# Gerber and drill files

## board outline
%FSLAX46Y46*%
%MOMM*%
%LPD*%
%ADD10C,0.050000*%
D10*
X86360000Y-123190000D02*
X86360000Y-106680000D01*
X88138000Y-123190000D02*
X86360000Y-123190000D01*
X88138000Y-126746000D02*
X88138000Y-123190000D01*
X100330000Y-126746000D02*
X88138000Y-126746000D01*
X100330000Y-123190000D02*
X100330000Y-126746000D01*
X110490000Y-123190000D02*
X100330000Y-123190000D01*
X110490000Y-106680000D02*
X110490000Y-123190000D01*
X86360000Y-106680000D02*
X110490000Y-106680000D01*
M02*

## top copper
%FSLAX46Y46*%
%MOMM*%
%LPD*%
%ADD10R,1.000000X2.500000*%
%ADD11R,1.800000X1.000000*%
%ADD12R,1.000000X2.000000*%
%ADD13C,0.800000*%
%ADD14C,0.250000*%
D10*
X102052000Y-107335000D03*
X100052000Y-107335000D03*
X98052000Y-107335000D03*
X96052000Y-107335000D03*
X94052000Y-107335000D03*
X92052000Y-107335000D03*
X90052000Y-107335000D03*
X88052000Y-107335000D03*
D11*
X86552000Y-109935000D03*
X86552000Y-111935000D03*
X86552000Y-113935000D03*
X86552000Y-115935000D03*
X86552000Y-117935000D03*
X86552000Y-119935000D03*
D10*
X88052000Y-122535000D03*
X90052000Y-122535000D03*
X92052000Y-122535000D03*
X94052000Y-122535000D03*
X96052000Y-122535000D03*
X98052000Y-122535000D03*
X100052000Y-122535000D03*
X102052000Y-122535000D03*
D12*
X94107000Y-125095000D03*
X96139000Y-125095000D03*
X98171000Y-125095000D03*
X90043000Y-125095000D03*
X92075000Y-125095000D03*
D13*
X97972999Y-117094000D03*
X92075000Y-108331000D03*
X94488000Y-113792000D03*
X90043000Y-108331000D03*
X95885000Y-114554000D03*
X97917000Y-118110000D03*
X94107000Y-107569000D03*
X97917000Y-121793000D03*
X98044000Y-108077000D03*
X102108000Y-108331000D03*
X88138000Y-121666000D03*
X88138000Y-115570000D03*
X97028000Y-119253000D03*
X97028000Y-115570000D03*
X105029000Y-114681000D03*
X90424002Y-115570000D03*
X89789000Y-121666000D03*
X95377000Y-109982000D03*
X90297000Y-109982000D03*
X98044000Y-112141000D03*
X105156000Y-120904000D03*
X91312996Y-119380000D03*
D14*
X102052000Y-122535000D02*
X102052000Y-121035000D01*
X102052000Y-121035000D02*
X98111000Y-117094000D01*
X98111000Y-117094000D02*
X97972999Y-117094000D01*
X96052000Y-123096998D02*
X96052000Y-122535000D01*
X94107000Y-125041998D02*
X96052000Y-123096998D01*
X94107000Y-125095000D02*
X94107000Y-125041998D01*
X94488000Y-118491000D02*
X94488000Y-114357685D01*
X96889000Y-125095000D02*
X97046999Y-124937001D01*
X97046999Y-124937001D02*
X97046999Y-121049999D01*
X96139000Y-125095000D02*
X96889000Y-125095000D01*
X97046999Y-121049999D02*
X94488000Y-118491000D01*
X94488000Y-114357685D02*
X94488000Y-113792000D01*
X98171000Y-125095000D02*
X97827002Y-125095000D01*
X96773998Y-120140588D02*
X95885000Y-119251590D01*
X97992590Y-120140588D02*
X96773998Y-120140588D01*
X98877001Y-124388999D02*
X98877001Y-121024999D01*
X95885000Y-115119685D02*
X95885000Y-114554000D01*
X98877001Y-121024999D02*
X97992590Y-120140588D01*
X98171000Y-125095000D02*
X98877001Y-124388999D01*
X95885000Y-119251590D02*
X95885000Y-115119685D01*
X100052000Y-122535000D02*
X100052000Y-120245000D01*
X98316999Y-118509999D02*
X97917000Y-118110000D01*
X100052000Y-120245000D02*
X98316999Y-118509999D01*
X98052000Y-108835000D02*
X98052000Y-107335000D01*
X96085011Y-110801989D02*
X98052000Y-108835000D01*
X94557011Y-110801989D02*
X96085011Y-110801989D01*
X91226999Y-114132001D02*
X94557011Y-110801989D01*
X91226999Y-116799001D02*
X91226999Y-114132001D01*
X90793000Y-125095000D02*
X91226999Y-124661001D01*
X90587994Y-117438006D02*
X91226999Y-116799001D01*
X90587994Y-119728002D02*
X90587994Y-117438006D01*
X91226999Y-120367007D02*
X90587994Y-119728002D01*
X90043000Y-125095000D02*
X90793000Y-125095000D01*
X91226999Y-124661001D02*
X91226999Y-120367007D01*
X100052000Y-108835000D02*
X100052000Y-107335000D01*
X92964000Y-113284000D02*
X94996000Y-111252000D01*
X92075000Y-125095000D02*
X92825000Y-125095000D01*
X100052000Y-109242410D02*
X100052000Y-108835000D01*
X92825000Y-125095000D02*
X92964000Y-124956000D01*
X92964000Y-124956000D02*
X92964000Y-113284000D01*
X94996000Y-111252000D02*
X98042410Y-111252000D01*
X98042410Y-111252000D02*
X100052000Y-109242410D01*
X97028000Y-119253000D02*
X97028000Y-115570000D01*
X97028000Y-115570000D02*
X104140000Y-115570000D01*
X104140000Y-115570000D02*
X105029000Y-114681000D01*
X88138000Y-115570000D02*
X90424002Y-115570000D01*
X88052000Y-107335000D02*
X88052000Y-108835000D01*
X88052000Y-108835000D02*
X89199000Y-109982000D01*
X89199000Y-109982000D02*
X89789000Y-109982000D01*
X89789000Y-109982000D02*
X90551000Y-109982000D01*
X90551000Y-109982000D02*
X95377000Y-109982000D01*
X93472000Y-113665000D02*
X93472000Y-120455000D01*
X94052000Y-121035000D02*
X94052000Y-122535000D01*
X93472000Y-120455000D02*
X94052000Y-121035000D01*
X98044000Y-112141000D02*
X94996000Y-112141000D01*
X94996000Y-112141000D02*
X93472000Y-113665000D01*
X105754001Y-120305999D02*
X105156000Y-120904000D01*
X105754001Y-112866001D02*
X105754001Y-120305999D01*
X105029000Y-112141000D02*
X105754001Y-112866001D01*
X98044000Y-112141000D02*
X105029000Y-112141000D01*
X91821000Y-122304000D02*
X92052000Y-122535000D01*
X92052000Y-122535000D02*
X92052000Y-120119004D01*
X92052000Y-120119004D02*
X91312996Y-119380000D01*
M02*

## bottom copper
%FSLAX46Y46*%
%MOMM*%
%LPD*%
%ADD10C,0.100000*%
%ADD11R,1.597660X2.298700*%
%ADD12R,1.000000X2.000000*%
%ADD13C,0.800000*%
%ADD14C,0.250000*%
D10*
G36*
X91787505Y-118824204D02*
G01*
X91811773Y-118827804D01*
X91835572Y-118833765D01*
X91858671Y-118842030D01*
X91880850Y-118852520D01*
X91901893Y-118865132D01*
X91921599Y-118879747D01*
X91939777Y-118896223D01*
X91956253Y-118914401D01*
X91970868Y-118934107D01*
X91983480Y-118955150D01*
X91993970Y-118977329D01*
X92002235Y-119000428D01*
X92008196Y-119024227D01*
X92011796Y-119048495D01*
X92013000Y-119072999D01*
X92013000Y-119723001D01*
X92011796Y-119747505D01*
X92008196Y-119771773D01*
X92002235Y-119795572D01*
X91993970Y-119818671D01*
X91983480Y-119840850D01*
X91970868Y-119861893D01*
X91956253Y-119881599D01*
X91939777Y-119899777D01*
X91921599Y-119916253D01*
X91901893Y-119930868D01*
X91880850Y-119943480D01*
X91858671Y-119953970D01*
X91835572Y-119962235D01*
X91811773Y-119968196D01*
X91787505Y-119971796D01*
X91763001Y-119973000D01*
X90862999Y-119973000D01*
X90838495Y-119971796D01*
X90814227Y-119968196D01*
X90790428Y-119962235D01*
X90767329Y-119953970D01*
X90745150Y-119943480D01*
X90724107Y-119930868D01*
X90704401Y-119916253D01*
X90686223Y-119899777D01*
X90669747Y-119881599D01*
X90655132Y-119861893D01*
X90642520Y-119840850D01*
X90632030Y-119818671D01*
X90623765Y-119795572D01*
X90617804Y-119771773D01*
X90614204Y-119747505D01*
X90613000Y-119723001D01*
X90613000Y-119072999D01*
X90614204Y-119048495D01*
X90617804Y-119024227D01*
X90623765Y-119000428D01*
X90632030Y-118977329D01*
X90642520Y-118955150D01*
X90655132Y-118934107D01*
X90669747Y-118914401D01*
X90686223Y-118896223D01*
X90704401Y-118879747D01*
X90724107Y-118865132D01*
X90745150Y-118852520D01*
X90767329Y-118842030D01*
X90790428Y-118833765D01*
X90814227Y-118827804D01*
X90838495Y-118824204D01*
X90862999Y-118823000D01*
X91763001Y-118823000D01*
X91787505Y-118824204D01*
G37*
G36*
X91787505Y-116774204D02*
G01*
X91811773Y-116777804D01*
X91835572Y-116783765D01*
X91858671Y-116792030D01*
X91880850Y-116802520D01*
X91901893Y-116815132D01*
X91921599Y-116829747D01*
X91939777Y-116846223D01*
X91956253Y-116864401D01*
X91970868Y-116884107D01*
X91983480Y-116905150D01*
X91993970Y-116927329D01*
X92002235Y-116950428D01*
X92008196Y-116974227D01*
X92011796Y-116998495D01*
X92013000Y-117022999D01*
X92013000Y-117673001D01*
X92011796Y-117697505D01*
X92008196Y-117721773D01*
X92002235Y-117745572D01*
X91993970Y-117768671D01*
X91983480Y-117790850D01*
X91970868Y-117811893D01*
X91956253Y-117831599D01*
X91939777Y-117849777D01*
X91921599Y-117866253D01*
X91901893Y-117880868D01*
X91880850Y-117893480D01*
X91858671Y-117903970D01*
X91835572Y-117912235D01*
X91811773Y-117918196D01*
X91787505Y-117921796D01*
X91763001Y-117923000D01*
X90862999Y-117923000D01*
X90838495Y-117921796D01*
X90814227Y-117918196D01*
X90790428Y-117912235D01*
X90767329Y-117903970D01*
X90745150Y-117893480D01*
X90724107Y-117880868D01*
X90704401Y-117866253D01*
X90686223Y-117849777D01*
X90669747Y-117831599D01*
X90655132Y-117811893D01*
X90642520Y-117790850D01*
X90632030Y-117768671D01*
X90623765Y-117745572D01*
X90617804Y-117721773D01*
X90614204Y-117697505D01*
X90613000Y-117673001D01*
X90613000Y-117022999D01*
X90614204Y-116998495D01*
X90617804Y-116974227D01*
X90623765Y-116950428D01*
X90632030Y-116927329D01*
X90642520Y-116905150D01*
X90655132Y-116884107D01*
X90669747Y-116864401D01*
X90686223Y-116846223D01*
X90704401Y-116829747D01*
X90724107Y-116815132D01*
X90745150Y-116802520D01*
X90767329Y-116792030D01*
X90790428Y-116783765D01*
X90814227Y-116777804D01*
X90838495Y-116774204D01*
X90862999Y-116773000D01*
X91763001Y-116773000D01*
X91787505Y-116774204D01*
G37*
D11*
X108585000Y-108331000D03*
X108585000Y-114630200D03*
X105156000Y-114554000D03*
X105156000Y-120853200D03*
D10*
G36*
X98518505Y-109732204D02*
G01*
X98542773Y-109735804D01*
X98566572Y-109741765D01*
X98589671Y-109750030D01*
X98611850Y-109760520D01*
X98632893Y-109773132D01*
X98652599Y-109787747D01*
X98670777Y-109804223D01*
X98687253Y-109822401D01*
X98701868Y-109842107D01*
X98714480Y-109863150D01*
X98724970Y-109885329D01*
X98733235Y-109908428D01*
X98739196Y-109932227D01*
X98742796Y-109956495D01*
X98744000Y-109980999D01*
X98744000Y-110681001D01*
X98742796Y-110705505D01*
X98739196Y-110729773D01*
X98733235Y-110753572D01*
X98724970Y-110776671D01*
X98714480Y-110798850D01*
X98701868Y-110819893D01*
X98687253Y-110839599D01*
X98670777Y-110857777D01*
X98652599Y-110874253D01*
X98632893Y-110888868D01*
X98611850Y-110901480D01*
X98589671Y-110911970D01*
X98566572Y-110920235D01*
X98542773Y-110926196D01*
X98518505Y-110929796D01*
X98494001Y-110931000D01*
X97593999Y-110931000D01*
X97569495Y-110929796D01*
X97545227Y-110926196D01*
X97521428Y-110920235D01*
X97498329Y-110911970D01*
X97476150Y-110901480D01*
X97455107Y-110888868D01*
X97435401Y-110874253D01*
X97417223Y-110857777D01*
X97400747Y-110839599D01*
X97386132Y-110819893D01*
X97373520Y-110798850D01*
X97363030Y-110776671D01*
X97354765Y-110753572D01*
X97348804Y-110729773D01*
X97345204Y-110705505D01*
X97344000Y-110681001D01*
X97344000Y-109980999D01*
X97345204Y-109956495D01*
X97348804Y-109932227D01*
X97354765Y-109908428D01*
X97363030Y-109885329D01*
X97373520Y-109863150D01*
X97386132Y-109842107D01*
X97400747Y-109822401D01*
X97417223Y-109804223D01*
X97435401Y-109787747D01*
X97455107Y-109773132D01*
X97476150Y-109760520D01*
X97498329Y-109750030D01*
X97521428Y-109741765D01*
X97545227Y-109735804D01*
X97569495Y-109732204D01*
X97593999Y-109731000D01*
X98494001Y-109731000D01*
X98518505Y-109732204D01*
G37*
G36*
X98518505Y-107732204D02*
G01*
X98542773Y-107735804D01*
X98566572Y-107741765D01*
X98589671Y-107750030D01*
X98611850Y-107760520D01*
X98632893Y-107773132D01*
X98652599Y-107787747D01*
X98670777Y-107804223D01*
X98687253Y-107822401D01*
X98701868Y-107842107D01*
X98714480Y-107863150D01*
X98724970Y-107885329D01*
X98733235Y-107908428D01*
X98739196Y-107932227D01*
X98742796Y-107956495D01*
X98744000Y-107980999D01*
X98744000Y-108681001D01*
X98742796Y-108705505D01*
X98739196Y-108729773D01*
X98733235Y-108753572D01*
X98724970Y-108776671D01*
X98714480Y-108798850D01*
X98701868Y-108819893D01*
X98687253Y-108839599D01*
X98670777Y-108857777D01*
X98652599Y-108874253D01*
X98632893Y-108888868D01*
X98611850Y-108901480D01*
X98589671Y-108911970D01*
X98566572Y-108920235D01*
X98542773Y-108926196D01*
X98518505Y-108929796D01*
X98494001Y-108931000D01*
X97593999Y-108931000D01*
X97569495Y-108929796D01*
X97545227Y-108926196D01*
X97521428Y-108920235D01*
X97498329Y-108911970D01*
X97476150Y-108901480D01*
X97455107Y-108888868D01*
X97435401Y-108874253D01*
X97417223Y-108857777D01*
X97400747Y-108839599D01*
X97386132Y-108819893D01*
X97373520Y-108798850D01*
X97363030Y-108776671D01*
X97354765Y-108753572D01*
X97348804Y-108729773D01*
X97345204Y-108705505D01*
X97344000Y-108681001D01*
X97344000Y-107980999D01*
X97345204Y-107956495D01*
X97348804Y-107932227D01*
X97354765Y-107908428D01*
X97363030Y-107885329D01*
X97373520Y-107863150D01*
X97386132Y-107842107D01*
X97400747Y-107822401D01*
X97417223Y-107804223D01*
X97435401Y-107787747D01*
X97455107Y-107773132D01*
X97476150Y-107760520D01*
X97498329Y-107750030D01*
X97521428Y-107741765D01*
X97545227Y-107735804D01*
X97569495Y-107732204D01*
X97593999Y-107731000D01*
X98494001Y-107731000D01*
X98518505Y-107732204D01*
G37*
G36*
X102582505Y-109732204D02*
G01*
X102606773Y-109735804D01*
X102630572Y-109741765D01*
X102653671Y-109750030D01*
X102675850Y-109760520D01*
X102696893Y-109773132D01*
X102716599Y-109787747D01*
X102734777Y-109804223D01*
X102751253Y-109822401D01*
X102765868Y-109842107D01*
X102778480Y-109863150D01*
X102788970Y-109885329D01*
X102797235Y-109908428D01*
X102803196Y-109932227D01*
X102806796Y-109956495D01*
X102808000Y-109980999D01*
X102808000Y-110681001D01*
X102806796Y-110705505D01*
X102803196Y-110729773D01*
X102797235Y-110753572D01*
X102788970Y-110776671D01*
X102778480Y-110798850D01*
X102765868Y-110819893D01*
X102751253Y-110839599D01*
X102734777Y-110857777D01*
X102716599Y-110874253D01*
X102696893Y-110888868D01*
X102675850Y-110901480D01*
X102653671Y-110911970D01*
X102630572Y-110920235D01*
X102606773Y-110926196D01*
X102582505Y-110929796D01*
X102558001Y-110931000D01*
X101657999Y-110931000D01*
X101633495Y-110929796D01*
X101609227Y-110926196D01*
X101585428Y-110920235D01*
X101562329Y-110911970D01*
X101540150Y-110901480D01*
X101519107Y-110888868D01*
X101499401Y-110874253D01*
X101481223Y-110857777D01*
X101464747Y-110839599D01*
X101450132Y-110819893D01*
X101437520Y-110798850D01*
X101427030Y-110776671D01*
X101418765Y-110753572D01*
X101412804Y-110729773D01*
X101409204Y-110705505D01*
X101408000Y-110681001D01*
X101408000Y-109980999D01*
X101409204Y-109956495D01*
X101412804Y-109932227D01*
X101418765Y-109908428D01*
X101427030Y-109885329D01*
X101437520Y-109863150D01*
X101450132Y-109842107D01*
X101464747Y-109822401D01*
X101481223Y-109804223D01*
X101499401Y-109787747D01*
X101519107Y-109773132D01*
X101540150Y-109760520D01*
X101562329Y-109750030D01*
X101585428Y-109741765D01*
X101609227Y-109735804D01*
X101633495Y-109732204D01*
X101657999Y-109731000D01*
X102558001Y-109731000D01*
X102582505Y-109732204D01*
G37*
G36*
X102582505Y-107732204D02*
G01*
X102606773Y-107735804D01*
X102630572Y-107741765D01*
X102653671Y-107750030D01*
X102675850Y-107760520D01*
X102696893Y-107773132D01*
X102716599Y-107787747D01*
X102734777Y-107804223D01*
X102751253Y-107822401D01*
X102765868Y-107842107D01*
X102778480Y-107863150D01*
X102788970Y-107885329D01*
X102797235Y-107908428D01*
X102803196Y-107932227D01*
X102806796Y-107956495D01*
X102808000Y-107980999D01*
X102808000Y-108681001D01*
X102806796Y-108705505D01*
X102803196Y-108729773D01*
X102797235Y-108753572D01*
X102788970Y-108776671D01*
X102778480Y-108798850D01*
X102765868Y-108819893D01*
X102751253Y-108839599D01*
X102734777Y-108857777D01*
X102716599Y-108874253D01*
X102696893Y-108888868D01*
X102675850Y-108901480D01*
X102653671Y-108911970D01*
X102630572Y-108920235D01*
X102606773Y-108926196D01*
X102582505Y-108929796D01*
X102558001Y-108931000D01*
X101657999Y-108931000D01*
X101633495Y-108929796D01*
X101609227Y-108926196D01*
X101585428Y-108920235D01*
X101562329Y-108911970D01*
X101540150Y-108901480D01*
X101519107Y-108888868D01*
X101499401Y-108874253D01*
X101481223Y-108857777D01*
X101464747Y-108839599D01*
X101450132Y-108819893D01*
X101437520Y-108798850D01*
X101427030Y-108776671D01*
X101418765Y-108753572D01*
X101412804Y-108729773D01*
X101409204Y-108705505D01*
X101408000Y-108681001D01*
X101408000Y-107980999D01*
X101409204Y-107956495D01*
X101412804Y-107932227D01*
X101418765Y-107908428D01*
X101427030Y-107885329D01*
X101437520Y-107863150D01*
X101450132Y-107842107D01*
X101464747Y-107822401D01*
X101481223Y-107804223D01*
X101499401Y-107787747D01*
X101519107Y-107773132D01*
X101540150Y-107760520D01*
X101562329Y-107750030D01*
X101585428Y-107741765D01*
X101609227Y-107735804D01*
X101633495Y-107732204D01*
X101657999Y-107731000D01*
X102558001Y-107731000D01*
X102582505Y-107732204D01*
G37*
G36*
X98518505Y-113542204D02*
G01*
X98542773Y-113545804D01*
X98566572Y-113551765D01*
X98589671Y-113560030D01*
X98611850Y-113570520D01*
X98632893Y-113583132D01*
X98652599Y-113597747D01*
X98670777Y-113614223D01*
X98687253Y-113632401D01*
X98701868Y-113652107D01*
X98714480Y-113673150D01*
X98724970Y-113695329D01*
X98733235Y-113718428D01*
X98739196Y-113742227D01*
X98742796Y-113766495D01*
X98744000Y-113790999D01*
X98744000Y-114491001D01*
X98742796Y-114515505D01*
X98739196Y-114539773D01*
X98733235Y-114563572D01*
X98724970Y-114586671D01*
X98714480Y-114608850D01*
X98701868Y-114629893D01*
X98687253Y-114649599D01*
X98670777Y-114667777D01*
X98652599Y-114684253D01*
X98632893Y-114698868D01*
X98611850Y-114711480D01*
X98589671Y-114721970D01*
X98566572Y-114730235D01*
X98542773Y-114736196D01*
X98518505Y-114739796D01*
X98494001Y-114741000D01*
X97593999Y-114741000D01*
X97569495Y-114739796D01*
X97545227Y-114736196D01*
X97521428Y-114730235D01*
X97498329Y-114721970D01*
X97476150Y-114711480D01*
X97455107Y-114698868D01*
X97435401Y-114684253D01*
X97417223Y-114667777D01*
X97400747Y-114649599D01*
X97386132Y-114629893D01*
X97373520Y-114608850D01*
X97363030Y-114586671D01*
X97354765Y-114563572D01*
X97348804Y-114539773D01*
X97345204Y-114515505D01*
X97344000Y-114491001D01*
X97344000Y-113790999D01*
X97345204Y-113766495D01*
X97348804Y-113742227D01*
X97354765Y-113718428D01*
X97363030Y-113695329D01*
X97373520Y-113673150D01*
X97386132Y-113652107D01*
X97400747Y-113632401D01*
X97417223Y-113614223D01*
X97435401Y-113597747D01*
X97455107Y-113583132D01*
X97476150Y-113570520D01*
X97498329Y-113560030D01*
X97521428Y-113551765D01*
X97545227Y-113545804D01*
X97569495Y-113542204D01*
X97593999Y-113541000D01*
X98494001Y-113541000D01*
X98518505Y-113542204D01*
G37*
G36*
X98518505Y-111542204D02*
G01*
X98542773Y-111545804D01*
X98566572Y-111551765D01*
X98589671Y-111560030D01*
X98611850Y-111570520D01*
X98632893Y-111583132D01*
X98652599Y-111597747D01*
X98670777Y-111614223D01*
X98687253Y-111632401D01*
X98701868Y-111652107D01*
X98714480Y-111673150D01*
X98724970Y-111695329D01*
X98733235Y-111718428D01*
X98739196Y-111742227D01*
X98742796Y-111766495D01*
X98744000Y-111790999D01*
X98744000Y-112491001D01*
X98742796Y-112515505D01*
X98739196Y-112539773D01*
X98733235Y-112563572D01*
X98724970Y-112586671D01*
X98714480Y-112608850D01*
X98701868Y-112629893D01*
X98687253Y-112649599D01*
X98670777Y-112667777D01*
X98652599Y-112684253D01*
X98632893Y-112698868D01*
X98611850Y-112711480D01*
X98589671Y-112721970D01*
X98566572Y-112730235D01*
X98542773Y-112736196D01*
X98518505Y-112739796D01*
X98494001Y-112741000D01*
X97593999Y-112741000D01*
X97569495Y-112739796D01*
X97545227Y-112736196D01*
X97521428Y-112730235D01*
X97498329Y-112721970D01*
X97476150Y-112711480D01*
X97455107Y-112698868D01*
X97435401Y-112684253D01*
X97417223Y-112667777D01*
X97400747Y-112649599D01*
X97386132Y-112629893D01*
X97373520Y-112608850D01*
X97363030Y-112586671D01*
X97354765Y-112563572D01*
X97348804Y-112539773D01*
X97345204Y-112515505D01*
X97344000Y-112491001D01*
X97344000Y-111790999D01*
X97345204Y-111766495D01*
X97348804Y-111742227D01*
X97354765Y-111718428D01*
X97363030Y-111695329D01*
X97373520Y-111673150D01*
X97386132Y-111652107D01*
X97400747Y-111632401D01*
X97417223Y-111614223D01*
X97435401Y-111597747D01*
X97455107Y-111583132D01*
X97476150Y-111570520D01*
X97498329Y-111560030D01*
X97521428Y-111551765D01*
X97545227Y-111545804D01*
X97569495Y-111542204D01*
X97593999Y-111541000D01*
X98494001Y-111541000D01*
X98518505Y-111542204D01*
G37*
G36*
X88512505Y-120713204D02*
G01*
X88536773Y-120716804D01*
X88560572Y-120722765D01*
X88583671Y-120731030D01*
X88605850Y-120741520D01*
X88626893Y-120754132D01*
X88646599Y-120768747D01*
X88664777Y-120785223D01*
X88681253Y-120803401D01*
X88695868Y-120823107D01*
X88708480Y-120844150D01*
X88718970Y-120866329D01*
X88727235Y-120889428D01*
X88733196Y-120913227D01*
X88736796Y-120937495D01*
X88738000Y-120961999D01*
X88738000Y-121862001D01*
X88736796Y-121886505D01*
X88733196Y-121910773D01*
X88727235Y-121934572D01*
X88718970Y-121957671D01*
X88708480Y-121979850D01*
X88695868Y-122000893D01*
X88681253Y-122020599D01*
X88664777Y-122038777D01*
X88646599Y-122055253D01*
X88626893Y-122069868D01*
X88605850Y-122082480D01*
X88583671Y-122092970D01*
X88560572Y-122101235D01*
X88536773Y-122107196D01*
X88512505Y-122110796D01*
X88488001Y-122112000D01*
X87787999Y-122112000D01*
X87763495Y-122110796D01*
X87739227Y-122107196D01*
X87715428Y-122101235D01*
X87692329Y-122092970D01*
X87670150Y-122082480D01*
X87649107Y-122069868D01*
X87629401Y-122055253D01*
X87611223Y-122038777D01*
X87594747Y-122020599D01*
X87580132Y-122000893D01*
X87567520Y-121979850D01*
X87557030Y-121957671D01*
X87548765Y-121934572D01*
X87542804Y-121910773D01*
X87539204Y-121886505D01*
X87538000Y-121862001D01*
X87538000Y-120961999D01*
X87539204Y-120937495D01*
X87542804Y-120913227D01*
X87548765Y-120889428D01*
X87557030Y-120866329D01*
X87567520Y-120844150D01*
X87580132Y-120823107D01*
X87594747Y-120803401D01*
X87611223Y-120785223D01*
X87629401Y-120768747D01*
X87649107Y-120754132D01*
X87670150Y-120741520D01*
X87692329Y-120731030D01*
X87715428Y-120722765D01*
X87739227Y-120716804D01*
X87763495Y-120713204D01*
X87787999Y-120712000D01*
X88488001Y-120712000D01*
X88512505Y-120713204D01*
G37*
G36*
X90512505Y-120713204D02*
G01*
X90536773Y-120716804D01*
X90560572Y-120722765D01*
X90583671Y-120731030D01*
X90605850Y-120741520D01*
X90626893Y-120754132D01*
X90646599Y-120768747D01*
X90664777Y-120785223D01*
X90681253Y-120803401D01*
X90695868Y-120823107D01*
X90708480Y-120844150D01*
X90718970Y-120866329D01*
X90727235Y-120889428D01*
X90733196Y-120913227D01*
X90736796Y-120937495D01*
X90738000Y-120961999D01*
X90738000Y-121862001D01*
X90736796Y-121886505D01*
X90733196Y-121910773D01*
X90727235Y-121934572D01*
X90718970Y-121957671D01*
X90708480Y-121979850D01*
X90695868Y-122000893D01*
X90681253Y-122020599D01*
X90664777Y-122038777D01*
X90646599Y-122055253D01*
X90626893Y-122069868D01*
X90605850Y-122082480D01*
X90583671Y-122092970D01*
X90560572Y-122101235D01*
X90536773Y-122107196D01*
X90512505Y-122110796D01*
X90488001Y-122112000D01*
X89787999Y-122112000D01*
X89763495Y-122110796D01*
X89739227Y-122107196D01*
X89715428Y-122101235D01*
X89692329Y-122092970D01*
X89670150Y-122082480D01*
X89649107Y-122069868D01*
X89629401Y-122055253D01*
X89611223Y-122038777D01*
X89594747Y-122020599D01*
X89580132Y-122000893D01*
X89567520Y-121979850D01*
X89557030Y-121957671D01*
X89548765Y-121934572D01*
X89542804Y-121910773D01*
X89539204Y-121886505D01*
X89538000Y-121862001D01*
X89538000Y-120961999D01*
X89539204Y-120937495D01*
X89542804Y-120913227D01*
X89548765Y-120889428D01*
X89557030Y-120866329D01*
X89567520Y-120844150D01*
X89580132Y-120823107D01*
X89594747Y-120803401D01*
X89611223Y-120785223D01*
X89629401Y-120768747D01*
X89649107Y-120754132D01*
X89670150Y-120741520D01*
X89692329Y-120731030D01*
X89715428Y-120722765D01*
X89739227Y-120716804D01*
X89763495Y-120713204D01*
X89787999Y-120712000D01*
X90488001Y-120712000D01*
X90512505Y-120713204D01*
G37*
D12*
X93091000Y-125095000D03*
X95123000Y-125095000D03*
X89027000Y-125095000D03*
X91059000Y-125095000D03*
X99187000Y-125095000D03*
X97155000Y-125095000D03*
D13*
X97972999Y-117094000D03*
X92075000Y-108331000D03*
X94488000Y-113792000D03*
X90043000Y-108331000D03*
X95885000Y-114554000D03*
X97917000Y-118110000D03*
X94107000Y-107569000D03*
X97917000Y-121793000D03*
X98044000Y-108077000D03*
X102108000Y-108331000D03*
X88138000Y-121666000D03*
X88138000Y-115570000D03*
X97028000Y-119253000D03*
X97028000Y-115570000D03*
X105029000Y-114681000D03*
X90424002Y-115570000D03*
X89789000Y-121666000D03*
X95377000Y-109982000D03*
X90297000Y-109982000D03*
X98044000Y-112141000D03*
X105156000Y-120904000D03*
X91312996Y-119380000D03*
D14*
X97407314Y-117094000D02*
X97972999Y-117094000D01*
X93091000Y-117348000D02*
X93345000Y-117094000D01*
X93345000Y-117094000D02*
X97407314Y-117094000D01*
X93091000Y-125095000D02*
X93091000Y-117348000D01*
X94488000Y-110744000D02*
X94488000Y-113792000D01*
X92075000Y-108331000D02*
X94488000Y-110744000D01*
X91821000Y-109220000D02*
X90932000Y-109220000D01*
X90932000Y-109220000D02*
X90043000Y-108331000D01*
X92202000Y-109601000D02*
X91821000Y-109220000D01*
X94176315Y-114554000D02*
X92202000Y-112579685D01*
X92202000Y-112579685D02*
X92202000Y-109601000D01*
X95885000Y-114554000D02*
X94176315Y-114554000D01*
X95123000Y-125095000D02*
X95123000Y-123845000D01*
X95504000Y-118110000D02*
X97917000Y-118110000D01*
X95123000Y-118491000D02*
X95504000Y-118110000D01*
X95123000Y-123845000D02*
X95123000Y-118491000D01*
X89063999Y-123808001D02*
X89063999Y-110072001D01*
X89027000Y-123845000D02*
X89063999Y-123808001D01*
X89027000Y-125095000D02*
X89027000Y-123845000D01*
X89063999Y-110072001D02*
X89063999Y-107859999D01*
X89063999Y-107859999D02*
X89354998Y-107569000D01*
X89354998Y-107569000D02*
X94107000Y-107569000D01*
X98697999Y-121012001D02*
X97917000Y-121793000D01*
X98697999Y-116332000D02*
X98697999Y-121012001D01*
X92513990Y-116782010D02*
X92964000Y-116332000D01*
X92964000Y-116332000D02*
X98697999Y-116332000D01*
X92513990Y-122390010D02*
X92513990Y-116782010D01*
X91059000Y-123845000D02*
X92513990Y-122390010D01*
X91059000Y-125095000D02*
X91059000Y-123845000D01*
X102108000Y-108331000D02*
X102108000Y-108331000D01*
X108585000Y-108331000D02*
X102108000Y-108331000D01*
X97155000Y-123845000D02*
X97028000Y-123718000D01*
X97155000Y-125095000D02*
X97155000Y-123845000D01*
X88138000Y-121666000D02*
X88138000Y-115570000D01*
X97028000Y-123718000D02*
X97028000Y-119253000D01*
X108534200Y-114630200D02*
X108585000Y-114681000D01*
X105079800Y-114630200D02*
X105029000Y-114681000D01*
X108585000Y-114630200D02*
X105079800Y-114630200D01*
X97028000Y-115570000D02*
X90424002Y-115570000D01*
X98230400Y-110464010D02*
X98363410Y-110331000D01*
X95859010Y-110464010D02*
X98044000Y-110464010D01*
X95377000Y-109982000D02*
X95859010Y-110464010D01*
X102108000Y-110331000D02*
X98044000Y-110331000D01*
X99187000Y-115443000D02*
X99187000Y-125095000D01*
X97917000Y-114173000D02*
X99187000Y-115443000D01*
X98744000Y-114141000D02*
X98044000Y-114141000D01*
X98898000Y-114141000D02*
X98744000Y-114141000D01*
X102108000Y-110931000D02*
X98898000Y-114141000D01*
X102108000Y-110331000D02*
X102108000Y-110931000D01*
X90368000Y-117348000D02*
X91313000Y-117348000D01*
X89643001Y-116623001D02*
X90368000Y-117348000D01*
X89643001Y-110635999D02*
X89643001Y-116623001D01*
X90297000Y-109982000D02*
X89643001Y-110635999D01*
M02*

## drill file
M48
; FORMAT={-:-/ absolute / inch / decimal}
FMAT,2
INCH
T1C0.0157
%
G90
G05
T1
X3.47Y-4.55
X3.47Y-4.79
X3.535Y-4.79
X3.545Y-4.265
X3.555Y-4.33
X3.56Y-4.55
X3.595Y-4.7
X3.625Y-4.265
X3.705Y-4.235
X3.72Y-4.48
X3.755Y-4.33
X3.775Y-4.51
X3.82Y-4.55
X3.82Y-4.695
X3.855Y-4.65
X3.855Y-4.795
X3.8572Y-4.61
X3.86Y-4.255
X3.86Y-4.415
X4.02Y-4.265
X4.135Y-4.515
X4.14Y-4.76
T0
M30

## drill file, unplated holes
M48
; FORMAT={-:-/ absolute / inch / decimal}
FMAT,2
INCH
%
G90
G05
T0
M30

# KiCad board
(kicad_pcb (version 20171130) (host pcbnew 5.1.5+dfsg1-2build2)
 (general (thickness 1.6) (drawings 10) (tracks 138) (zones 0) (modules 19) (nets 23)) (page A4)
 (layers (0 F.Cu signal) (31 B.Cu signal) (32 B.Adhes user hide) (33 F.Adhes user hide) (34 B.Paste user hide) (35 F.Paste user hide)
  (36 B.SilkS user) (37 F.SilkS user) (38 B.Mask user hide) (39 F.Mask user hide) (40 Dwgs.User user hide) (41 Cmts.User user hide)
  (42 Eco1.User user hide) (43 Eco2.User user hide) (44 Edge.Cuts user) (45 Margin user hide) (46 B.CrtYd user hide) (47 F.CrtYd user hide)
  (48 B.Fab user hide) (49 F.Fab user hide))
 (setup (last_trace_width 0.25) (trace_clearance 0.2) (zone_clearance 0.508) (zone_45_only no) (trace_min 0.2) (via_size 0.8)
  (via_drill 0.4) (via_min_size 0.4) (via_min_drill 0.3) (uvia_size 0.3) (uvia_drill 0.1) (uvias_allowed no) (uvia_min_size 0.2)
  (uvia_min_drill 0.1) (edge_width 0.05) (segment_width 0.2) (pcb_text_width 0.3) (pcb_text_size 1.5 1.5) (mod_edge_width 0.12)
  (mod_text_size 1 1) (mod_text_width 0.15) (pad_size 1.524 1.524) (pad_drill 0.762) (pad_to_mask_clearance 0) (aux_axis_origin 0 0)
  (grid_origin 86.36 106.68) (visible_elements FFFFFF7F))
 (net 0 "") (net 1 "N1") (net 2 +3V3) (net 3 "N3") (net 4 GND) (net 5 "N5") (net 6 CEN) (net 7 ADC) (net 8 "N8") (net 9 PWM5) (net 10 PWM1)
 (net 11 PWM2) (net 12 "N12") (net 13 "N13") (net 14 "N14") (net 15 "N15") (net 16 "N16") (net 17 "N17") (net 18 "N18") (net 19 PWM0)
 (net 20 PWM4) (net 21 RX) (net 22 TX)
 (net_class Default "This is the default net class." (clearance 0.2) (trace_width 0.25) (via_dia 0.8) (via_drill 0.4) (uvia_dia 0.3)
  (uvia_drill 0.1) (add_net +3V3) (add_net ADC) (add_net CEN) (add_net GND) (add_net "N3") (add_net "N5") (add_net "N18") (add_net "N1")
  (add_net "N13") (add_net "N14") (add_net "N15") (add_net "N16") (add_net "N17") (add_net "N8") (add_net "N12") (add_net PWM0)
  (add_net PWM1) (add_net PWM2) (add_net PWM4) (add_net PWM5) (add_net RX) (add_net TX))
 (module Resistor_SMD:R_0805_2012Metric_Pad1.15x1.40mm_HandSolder (layer B.Cu) (at 91.313 118.373 270)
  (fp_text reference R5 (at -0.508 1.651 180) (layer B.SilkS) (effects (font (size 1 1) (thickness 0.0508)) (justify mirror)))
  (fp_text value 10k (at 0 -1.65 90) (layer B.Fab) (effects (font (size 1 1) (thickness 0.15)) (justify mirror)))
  (pad 2 smd roundrect (at 1.025 0 270) (size 1.15 1.4) (layers B.Cu B.Paste B.Mask) (roundrect_rratio 0.217391) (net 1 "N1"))
  (pad 1 smd roundrect (at -1.025 0 270) (size 1.15 1.4) (layers B.Cu B.Paste B.Mask) (roundrect_rratio 0.217391) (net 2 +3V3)))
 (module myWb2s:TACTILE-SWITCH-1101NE (layer B.Cu) (at 108.585 111.4806 90)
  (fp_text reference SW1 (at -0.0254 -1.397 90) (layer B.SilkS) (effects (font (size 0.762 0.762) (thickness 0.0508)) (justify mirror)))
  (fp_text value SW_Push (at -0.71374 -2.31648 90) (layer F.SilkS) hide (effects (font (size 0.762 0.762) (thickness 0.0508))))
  (pad 2 smd rect (at 3.1496 0 270) (size 2.2987 1.59766) (layers B.Cu B.Paste B.Mask) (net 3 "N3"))
  (pad 1 smd rect (at -3.1496 0 270) (size 2.2987 1.59766) (layers B.Cu B.Paste B.Mask) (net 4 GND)))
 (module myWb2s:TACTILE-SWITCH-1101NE (layer B.Cu) (at 105.156 117.7036 270)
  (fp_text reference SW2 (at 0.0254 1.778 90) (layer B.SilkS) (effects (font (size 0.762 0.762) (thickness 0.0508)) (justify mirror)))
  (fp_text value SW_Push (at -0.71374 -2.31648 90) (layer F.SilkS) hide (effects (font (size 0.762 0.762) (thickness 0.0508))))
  (pad 1 smd rect (at -3.1496 0 90) (size 2.2987 1.59766) (layers B.Cu B.Paste B.Mask) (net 4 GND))
  (pad 2 smd rect (at 3.1496 0 90) (size 2.2987 1.59766) (layers B.Cu B.Paste B.Mask) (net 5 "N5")))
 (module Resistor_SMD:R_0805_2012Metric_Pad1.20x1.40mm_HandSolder (layer B.Cu) (at 98.044 109.331 270)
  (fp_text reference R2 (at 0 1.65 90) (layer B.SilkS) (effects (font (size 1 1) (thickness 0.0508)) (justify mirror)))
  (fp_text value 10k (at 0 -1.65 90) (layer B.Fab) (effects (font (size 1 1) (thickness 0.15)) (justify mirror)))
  (pad 2 smd roundrect (at 1 0 270) (size 1.2 1.4) (layers B.Cu B.Paste B.Mask) (roundrect_rratio 0.208333) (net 2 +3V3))
  (pad 1 smd roundrect (at -1 0 270) (size 1.2 1.4) (layers B.Cu B.Paste B.Mask) (roundrect_rratio 0.208333) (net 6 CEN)))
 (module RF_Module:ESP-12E (layer F.Cu) (at 98.552 114.935 270)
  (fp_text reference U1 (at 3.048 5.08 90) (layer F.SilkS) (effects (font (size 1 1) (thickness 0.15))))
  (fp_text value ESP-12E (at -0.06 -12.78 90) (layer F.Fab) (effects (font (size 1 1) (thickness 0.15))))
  (pad 1 smd rect (at -7.6 -3.5 270) (size 2.5 1) (layers F.Cu F.Paste F.Mask) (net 3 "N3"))
  (pad 2 smd rect (at -7.6 -1.5 270) (size 2.5 1) (layers F.Cu F.Paste F.Mask) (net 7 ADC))
  (pad 3 smd rect (at -7.6 0.5 270) (size 2.5 1) (layers F.Cu F.Paste F.Mask) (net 6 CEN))
  (pad 4 smd rect (at -7.6 2.5 270) (size 2.5 1) (layers F.Cu F.Paste F.Mask) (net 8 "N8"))
  (pad 5 smd rect (at -7.6 4.5 270) (size 2.5 1) (layers F.Cu F.Paste F.Mask) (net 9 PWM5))
  (pad 6 smd rect (at -7.6 6.5 270) (size 2.5 1) (layers F.Cu F.Paste F.Mask) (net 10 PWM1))
  (pad 7 smd rect (at -7.6 8.5 270) (size 2.5 1) (layers F.Cu F.Paste F.Mask) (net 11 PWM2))
  (pad 8 smd rect (at -7.6 10.5 270) (size 2.5 1) (layers F.Cu F.Paste F.Mask) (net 2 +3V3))
  (pad 9 smd rect (at -5 12 270) (size 1 1.8) (layers F.Cu F.Paste F.Mask) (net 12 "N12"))
  (pad 10 smd rect (at -3 12 270) (size 1 1.8) (layers F.Cu F.Paste F.Mask) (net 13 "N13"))
  (pad 11 smd rect (at -1 12 270) (size 1 1.8) (layers F.Cu F.Paste F.Mask) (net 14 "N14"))
  (pad 12 smd rect (at 1 12 270) (size 1 1.8) (layers F.Cu F.Paste F.Mask) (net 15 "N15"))
  (pad 13 smd rect (at 3 12 270) (size 1 1.8) (layers F.Cu F.Paste F.Mask) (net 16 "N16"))
  (pad 14 smd rect (at 5 12 270) (size 1 1.8) (layers F.Cu F.Paste F.Mask) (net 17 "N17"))
  (pad 15 smd rect (at 7.6 10.5 270) (size 2.5 1) (layers F.Cu F.Paste F.Mask) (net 4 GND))
  (pad 16 smd rect (at 7.6 8.5 270) (size 2.5 1) (layers F.Cu F.Paste F.Mask) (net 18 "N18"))
  (pad 17 smd rect (at 7.6 6.5 270) (size 2.5 1) (layers F.Cu F.Paste F.Mask) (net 1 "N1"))
  (pad 18 smd rect (at 7.6 4.5 270) (size 2.5 1) (layers F.Cu F.Paste F.Mask) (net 5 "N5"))
  (pad 19 smd rect (at 7.6 2.5 270) (size 2.5 1) (layers F.Cu F.Paste F.Mask) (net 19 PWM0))
  (pad 20 smd rect (at 7.6 0.5 270) (size 2.5 1) (layers F.Cu F.Paste F.Mask) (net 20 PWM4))
  (pad 21 smd rect (at 7.6 -1.5 270) (size 2.5 1) (layers F.Cu F.Paste F.Mask) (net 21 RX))
  (pad 22 smd rect (at 7.6 -3.5 270) (size 2.5 1) (layers F.Cu F.Paste F.Mask) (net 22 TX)))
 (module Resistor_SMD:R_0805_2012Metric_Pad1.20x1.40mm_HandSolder (layer B.Cu) (at 102.108 109.331 270)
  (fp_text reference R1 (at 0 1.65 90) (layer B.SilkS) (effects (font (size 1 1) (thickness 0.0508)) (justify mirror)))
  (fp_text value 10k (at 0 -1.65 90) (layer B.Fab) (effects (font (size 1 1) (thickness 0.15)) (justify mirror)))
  (pad 2 smd roundrect (at 1 0 270) (size 1.2 1.4) (layers B.Cu B.Paste B.Mask) (roundrect_rratio 0.208333) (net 2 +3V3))
  (pad 1 smd roundrect (at -1 0 270) (size 1.2 1.4) (layers B.Cu B.Paste B.Mask) (roundrect_rratio 0.208333) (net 3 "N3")))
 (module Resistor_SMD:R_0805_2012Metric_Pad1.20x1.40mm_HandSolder (layer B.Cu) (at 98.044 113.141 270)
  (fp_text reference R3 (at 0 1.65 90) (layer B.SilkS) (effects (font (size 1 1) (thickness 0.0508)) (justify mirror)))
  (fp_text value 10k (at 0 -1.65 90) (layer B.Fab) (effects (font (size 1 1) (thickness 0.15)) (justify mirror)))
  (pad 2 smd roundrect (at 1 0 270) (size 1.2 1.4) (layers B.Cu B.Paste B.Mask) (roundrect_rratio 0.208333) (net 2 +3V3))
  (pad 1 smd roundrect (at -1 0 270) (size 1.2 1.4) (layers B.Cu B.Paste B.Mask) (roundrect_rratio 0.208333) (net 5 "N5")))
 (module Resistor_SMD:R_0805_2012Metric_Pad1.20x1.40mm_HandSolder (layer B.Cu) (at 89.138 121.412)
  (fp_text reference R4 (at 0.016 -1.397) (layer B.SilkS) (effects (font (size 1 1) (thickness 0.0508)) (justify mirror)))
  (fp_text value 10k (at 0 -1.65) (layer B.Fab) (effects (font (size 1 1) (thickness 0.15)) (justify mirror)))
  (pad 1 smd roundrect (at -1 0) (size 1.2 1.4) (layers B.Cu B.Paste B.Mask) (roundrect_rratio 0.208333) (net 4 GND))
  (pad 2 smd roundrect (at 1 0) (size 1.2 1.4) (layers B.Cu B.Paste B.Mask) (roundrect_rratio 0.208333) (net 18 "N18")))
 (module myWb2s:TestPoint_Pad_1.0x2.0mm (layer B.Cu) (at 93.091 125.095)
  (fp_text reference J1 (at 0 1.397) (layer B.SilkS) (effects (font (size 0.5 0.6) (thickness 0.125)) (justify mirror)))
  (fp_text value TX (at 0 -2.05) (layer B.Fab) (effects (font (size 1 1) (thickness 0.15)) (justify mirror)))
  (pad 1 smd rect (at 0 0) (size 1 2) (layers B.Cu B.Mask) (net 22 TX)))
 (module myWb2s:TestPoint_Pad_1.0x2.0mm (layer F.Cu) (at 94.107 125.095)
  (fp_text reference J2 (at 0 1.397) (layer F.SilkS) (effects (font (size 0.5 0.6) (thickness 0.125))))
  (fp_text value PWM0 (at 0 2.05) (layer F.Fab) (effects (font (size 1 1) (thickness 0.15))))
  (pad 1 smd rect (at 0 0) (size 1 2) (layers F.Cu F.Mask) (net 19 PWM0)))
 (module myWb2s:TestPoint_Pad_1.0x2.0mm (layer F.Cu) (at 96.139 125.095)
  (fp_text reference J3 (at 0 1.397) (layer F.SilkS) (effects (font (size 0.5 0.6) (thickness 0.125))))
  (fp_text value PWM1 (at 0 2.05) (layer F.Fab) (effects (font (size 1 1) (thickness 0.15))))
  (pad 1 smd rect (at 0 0) (size 1 2) (layers F.Cu F.Mask) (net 10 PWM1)))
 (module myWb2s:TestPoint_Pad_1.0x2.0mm (layer F.Cu) (at 98.171 125.095)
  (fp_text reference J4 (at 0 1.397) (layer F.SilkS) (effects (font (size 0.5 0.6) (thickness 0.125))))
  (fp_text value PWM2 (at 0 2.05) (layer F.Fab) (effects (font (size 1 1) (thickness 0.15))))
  (pad 1 smd rect (at 0 0) (size 1 2) (layers F.Cu F.Mask) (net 11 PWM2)))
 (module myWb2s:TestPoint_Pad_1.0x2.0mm (layer B.Cu) (at 95.123 125.095)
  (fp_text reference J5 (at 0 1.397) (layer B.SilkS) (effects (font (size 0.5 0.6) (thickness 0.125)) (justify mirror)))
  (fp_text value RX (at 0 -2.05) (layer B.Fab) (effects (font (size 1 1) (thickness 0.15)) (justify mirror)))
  (pad 1 smd rect (at 0 0) (size 1 2) (layers B.Cu B.Mask) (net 21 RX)))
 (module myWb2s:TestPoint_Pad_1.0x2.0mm (layer B.Cu) (at 89.027 125.095)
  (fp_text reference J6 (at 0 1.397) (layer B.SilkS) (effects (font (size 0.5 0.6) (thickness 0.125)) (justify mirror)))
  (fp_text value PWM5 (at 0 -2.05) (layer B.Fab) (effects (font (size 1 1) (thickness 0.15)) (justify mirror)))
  (pad 1 smd rect (at 0 0) (size 1 2) (layers B.Cu B.Mask) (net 9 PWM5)))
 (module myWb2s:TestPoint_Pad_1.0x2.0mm (layer B.Cu) (at 91.059 125.095)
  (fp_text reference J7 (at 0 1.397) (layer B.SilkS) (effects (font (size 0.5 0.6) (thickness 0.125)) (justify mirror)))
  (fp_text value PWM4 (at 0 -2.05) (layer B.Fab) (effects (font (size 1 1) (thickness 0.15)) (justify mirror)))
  (pad 1 smd rect (at 0 0) (size 1 2) (layers B.Cu B.Mask) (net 20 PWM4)))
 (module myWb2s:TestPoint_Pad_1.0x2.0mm (layer F.Cu) (at 90.043 125.095)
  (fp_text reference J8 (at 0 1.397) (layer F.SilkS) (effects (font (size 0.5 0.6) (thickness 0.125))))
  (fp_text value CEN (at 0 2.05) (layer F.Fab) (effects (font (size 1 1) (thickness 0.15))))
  (pad 1 smd rect (at 0 0) (size 1 2) (layers F.Cu F.Mask) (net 6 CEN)))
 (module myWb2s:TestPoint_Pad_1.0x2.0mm (layer F.Cu) (at 92.075 125.095)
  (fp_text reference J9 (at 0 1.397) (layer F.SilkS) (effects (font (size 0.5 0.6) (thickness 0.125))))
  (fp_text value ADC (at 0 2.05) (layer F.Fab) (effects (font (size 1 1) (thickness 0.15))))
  (pad 1 smd rect (at 0 0) (size 1 2) (layers F.Cu F.Mask) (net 7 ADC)))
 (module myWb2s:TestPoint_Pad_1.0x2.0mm (layer B.Cu) (at 99.187 125.095)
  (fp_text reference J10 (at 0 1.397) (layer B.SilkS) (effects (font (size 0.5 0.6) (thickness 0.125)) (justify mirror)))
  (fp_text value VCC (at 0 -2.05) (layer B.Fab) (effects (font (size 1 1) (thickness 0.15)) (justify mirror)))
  (pad 1 smd rect (at 0 0) (size 1 2) (layers B.Cu B.Mask) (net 2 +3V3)))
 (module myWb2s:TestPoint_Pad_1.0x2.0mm (layer B.Cu) (at 97.155 125.095)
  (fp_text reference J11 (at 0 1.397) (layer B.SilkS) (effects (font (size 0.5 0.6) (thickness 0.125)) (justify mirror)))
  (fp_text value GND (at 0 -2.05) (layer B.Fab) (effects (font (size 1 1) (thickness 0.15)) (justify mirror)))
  (pad 1 smd rect (at 0 0) (size 1 2) (layers B.Cu B.Mask) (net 4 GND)))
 (gr_line (start 86.36 123.19) (end 86.36 106.68) (layer Edge.Cuts) (width 0.05))
 (gr_line (start 88.138 123.19) (end 86.36 123.19) (layer Edge.Cuts) (width 0.05))
 (gr_line (start 88.138 126.746) (end 88.138 123.19) (layer Edge.Cuts) (width 0.05))
 (gr_line (start 100.33 126.746) (end 88.138 126.746) (layer Edge.Cuts) (width 0.05))
 (gr_line (start 100.33 123.19) (end 100.33 126.746) (layer Edge.Cuts) (width 0.05))
 (gr_line (start 110.49 123.19) (end 100.33 123.19) (layer Edge.Cuts) (width 0.05))
 (gr_line (start 110.49 106.68) (end 110.49 123.19) (layer Edge.Cuts) (width 0.05))
 (gr_line (start 86.36 106.68) (end 110.49 106.68) (layer Edge.Cuts) (width 0.05))
 (via (at 97.972999 117.094) (size 0.8) (drill 0.4) (layers F.Cu B.Cu) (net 22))
 (segment (start 102.052 122.535) (end 102.052 121.035) (width 0.25) (layer F.Cu) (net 22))
 (segment (start 102.052 121.035) (end 98.111 117.094) (width 0.25) (layer F.Cu) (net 22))
 (segment (start 98.111 117.094) (end 97.972999 117.094) (width 0.25) (layer F.Cu) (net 22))
 (segment (start 97.407314 117.094) (end 97.972999 117.094) (width 0.25) (layer B.Cu) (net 22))
 (segment (start 93.091 117.348) (end 93.345 117.094) (width 0.25) (layer B.Cu) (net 22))
 (segment (start 93.345 117.094) (end 97.407314 117.094) (width 0.25) (layer B.Cu) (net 22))
 (segment (start 93.091 125.095) (end 93.091 117.348) (width 0.25) (layer B.Cu) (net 22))
 (segment (start 96.052 123.096998) (end 96.052 122.535) (width 0.25) (layer F.Cu) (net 19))
 (segment (start 94.107 125.041998) (end 96.052 123.096998) (width 0.25) (layer F.Cu) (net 19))
 (segment (start 94.107 125.095) (end 94.107 125.041998) (width 0.25) (layer F.Cu) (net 19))
 (via (at 92.075 108.331) (size 0.8) (drill 0.4) (layers F.Cu B.Cu) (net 10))
 (via (at 94.488 113.792) (size 0.8) (drill 0.4) (layers F.Cu B.Cu) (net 10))
 (segment (start 94.488 118.491) (end 94.488 114.357685) (width 0.25) (layer F.Cu) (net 10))
 (segment (start 96.889 125.095) (end 97.046999 124.937001) (width 0.25) (layer F.Cu) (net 10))
 (segment (start 97.046999 124.937001) (end 97.046999 121.049999) (width 0.25) (layer F.Cu) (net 10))
 (segment (start 96.139 125.095) (end 96.889 125.095) (width 0.25) (layer F.Cu) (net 10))
 (segment (start 94.488 110.744) (end 94.488 113.792) (width 0.25) (layer B.Cu) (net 10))
 (segment (start 97.046999 121.049999) (end 94.488 118.491) (width 0.25) (layer F.Cu) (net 10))
 (segment (start 92.075 108.331) (end 94.488 110.744) (width 0.25) (layer B.Cu) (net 10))
 (segment (start 94.488 114.357685) (end 94.488 113.792) (width 0.25) (layer F.Cu) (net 10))
 (via (at 90.043 108.331) (size 0.8) (drill 0.4) (layers F.Cu B.Cu) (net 11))
 (segment (start 98.171 125.095) (end 97.827002 125.095) (width 0.25) (layer F.Cu) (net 11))
 (via (at 95.885 114.554) (size 0.8) (drill 0.4) (layers F.Cu B.Cu) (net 11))
 (segment (start 96.773998 120.140588) (end 95.885 119.25159) (width 0.25) (layer F.Cu) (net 11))
 (segment (start 97.99259 120.140588) (end 96.773998 120.140588) (width 0.25) (layer F.Cu) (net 11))
 (segment (start 98.877001 124.388999) (end 98.877001 121.024999) (width 0.25) (layer F.Cu) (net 11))
 (segment (start 95.885 115.119685) (end 95.885 114.554) (width 0.25) (layer F.Cu) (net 11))
 (segment (start 98.877001 121.024999) (end 97.99259 120.140588) (width 0.25) (layer F.Cu) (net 11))
 (segment (start 98.171 125.095) (end 98.877001 124.388999) (width 0.25) (layer F.Cu) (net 11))
 (segment (start 95.885 119.25159) (end 95.885 115.119685) (width 0.25) (layer F.Cu) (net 11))
 (segment (start 91.821 109.22) (end 90.932 109.22) (width 0.25) (layer B.Cu) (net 11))
 (segment (start 90.932 109.22) (end 90.043 108.331) (width 0.25) (layer B.Cu) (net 11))
 (segment (start 92.202 109.601) (end 91.821 109.22) (width 0.25) (layer B.Cu) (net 11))
 (segment (start 94.176315 114.554) (end 92.202 112.579685) (width 0.25) (layer B.Cu) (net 11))
 (segment (start 92.202 112.579685) (end 92.202 109.601) (width 0.25) (layer B.Cu) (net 11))
 (segment (start 95.885 114.554) (end 94.176315 114.554) (width 0.25) (layer B.Cu) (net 11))
 (segment (start 95.123 125.095) (end 95.123 123.845) (width 0.25) (layer B.Cu) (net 21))
 (via (at 97.917 118.11) (size 0.8) (drill 0.4) (layers F.Cu B.Cu) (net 21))
 (segment (start 100.052 122.535) (end 100.052 120.245) (width 0.25) (layer F.Cu) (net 21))
 (segment (start 98.316999 118.509999) (end 97.917 118.11) (width 0.25) (layer F.Cu) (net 21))
 (segment (start 100.052 120.245) (end 98.316999 118.509999) (width 0.25) (layer F.Cu) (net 21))
 (segment (start 95.504 118.11) (end 97.917 118.11) (width 0.25) (layer B.Cu) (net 21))
 (segment (start 95.123 118.491) (end 95.504 118.11) (width 0.25) (layer B.Cu) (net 21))
 (segment (start 95.123 123.845) (end 95.123 118.491) (width 0.25) (layer B.Cu) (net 21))
 (segment (start 89.063999 123.808001) (end 89.063999 110.072001) (width 0.25) (layer B.Cu) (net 9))
 (segment (start 89.027 123.845) (end 89.063999 123.808001) (width 0.25) (layer B.Cu) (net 9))
 (segment (start 89.027 125.095) (end 89.027 123.845) (width 0.25) (layer B.Cu) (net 9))
 (segment (start 89.063999 110.072001) (end 89.063999 107.859999) (width 0.25) (layer B.Cu) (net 9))
 (segment (start 89.063999 107.859999) (end 89.354998 107.569) (width 0.25) (layer B.Cu) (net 9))
 (segment (start 89.354998 107.569) (end 94.107 107.569) (width 0.25) (layer B.Cu) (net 9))
 (via (at 94.107 107.569) (size 0.8) (drill 0.4) (layers F.Cu B.Cu) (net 9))
 (via (at 97.917 121.793) (size 0.8) (drill 0.4) (layers F.Cu B.Cu) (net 20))
 (segment (start 98.697999 121.012001) (end 97.917 121.793) (width 0.25) (layer B.Cu) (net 20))
 (segment (start 98.697999 116.332) (end 98.697999 121.012001) (width 0.25) (layer B.Cu) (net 20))
 (segment (start 92.51399 116.78201) (end 92.964 116.332) (width 0.25) (layer B.Cu) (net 20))
 (segment (start 92.964 116.332) (end 98.697999 116.332) (width 0.25) (layer B.Cu) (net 20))
 (segment (start 92.51399 122.39001) (end 92.51399 116.78201) (width 0.25) (layer B.Cu) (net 20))
 (segment (start 91.059 123.845) (end 92.51399 122.39001) (width 0.25) (layer B.Cu) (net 20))
 (segment (start 91.059 125.095) (end 91.059 123.845) (width 0.25) (layer B.Cu) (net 20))
 (via (at 98.044 108.077) (size 0.8) (drill 0.4) (layers F.Cu B.Cu) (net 6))
 (segment (start 98.052 108.835) (end 98.052 107.335) (width 0.25) (layer F.Cu) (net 6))
 (segment (start 96.085011 110.801989) (end 98.052 108.835) (width 0.25) (layer F.Cu) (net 6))
 (segment (start 94.557011 110.801989) (end 96.085011 110.801989) (width 0.25) (layer F.Cu) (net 6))
 (segment (start 91.226999 114.132001) (end 94.557011 110.801989) (width 0.25) (layer F.Cu) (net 6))
 (segment (start 91.226999 116.799001) (end 91.226999 114.132001) (width 0.25) (layer F.Cu) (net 6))
 (segment (start 90.793 125.095) (end 91.226999 124.661001) (width 0.25) (layer F.Cu) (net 6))
 (segment (start 90.587994 117.438006) (end 91.226999 116.799001) (width 0.25) (layer F.Cu) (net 6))
 (segment (start 90.587994 119.728002) (end 90.587994 117.438006) (width 0.25) (layer F.Cu) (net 6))
 (segment (start 91.226999 120.367007) (end 90.587994 119.728002) (width 0.25) (layer F.Cu) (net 6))
 (segment (start 90.043 125.095) (end 90.793 125.095) (width 0.25) (layer F.Cu) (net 6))
 (segment (start 91.226999 124.661001) (end 91.226999 120.367007) (width 0.25) (layer F.Cu) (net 6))
 (segment (start 100.052 108.835) (end 100.052 107.335) (width 0.25) (layer F.Cu) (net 7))
 (segment (start 92.964 113.284) (end 94.996 111.252) (width 0.25) (layer F.Cu) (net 7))
 (segment (start 92.075 125.095) (end 92.825 125.095) (width 0.25) (layer F.Cu) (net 7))
 (segment (start 100.052 109.24241) (end 100.052 108.835) (width 0.25) (layer F.Cu) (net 7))
 (segment (start 92.825 125.095) (end 92.964 124.956) (width 0.25) (layer F.Cu) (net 7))
 (segment (start 92.964 124.956) (end 92.964 113.284) (width 0.25) (layer F.Cu) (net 7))
 (segment (start 94.996 111.252) (end 98.04241 111.252) (width 0.25) (layer F.Cu) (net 7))
 (segment (start 98.04241 111.252) (end 100.052 109.24241) (width 0.25) (layer F.Cu) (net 7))
 (segment (start 102.108 108.331) (end 102.108 108.331) (width 0.25) (layer B.Cu) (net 3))
 (via (at 102.108 108.331) (size 0.8) (drill 0.4) (layers F.Cu B.Cu) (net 3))
 (segment (start 108.585 108.331) (end 102.108 108.331) (width 0.25) (layer B.Cu) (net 3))
 (via (at 88.138 121.666) (size 0.8) (drill 0.4) (layers F.Cu B.Cu) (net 4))
 (segment (start 97.155 123.845) (end 97.028 123.718) (width 0.25) (layer B.Cu) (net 4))
 (segment (start 97.155 125.095) (end 97.155 123.845) (width 0.25) (layer B.Cu) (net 4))
 (segment (start 88.138 121.666) (end 88.138 115.57) (width 0.25) (layer B.Cu) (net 4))
 (via (at 88.138 115.57) (size 0.8) (drill 0.4) (layers F.Cu B.Cu) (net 4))
 (segment (start 97.028 123.718) (end 97.028 119.253) (width 0.25) (layer B.Cu) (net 4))
 (via (at 97.028 119.253) (size 0.8) (drill 0.4) (layers F.Cu B.Cu) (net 4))
 (via (at 97.028 115.57) (size 0.8) (drill 0.4) (layers F.Cu B.Cu) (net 4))
 (segment (start 97.028 119.253) (end 97.028 115.57) (width 0.25) (layer F.Cu) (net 4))
 (segment (start 108.5342 114.6302) (end 108.585 114.681) (width 0.25) (layer B.Cu) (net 4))
 (segment (start 97.028 115.57) (end 104.14 115.57) (width 0.25) (layer F.Cu) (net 4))
 (segment (start 104.14 115.57) (end 105.029 114.681) (width 0.25) (layer F.Cu) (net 4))
 (via (at 105.029 114.681) (size 0.8) (drill 0.4) (layers F.Cu B.Cu) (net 4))
 (segment (start 105.0798 114.6302) (end 105.029 114.681) (width 0.25) (layer B.Cu) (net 4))
 (segment (start 108.585 114.6302) (end 105.0798 114.6302) (width 0.25) (layer B.Cu) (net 4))
 (via (at 90.424002 115.57) (size 0.8) (drill 0.4) (layers F.Cu B.Cu) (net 4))
 (segment (start 97.028 115.57) (end 90.424002 115.57) (width 0.25) (layer B.Cu) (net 4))
 (segment (start 88.138 115.57) (end 90.424002 115.57) (width 0.25) (layer F.Cu) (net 4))
 (via (at 89.789 121.666) (size 0.8) (drill 0.4) (layers F.Cu B.Cu) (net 18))
 (segment (start 98.2304 110.46401) (end 98.36341 110.331) (width 0.25) (layer B.Cu) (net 2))
 (via (at 95.377 109.982) (size 0.8) (drill 0.4) (layers F.Cu B.Cu) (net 2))
 (segment (start 95.85901 110.46401) (end 98.044 110.46401) (width 0.25) (layer B.Cu) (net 2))
 (segment (start 95.377 109.982) (end 95.85901 110.46401) (width 0.25) (layer B.Cu) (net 2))
 (segment (start 88.052 107.335) (end 88.052 108.835) (width 0.25) (layer F.Cu) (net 2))
 (segment (start 88.052 108.835) (end 89.199 109.982) (width 0.25) (layer F.Cu) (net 2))
 (segment (start 89.199 109.982) (end 89.789 109.982) (width 0.25) (layer F.Cu) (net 2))
 (segment (start 102.108 110.331) (end 98.044 110.331) (width 0.25) (layer B.Cu) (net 2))
 (segment (start 99.187 115.443) (end 99.187 125.095) (width 0.25) (layer B.Cu) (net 2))
 (segment (start 97.917 114.173) (end 99.187 115.443) (width 0.25) (layer B.Cu) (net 2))
 (segment (start 98.744 114.141) (end 98.044 114.141) (width 0.25) (layer B.Cu) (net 2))
 (segment (start 98.898 114.141) (end 98.744 114.141) (width 0.25) (layer B.Cu) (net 2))
 (segment (start 102.108 110.931) (end 98.898 114.141) (width 0.25) (layer B.Cu) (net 2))
 (segment (start 102.108 110.331) (end 102.108 110.931) (width 0.25) (layer B.Cu) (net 2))
 (segment (start 89.789 109.982) (end 90.551 109.982) (width 0.25) (layer F.Cu) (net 2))
 (segment (start 90.551 109.982) (end 95.377 109.982) (width 0.25) (layer F.Cu) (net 2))
 (via (at 90.297 109.982) (size 0.8) (drill 0.4) (layers F.Cu B.Cu) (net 2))
 (segment (start 90.368 117.348) (end 91.313 117.348) (width 0.25) (layer B.Cu) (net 2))
 (segment (start 89.643001 116.623001) (end 90.368 117.348) (width 0.25) (layer B.Cu) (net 2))
 (segment (start 89.643001 110.635999) (end 89.643001 116.623001) (width 0.25) (layer B.Cu) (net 2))
 (segment (start 90.297 109.982) (end 89.643001 110.635999) (width 0.25) (layer B.Cu) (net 2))
 (segment (start 93.472 113.665) (end 93.472 120.455) (width 0.25) (layer F.Cu) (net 5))
 (via (at 98.044 112.141) (size 0.8) (drill 0.4) (layers F.Cu B.Cu) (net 5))
 (segment (start 94.052 121.035) (end 94.052 122.535) (width 0.25) (layer F.Cu) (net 5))
 (segment (start 93.472 120.455) (end 94.052 121.035) (width 0.25) (layer F.Cu) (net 5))
 (segment (start 98.044 112.141) (end 94.996 112.141) (width 0.25) (layer F.Cu) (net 5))
 (segment (start 94.996 112.141) (end 93.472 113.665) (width 0.25) (layer F.Cu) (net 5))
 (via (at 105.156 120.904) (size 0.8) (drill 0.4) (layers F.Cu B.Cu) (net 5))
 (segment (start 105.754001 120.305999) (end 105.156 120.904) (width 0.25) (layer F.Cu) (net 5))
 (segment (start 105.754001 112.866001) (end 105.754001 120.305999) (width 0.25) (layer F.Cu) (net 5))
 (segment (start 105.029 112.141) (end 105.754001 112.866001) (width 0.25) (layer F.Cu) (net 5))
 (segment (start 98.044 112.141) (end 105.029 112.141) (width 0.25) (layer F.Cu) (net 5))
 (segment (start 91.821 122.304) (end 92.052 122.535) (width 0.25) (layer F.Cu) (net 1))
 (via (at 91.312996 119.38) (size 0.8) (drill 0.4) (layers F.Cu B.Cu) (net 1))
 (segment (start 92.052 122.535) (end 92.052 120.119004) (width 0.25) (layer F.Cu) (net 1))
 (segment (start 92.052 120.119004) (end 91.312996 119.38) (width 0.25) (layer F.Cu) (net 1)))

